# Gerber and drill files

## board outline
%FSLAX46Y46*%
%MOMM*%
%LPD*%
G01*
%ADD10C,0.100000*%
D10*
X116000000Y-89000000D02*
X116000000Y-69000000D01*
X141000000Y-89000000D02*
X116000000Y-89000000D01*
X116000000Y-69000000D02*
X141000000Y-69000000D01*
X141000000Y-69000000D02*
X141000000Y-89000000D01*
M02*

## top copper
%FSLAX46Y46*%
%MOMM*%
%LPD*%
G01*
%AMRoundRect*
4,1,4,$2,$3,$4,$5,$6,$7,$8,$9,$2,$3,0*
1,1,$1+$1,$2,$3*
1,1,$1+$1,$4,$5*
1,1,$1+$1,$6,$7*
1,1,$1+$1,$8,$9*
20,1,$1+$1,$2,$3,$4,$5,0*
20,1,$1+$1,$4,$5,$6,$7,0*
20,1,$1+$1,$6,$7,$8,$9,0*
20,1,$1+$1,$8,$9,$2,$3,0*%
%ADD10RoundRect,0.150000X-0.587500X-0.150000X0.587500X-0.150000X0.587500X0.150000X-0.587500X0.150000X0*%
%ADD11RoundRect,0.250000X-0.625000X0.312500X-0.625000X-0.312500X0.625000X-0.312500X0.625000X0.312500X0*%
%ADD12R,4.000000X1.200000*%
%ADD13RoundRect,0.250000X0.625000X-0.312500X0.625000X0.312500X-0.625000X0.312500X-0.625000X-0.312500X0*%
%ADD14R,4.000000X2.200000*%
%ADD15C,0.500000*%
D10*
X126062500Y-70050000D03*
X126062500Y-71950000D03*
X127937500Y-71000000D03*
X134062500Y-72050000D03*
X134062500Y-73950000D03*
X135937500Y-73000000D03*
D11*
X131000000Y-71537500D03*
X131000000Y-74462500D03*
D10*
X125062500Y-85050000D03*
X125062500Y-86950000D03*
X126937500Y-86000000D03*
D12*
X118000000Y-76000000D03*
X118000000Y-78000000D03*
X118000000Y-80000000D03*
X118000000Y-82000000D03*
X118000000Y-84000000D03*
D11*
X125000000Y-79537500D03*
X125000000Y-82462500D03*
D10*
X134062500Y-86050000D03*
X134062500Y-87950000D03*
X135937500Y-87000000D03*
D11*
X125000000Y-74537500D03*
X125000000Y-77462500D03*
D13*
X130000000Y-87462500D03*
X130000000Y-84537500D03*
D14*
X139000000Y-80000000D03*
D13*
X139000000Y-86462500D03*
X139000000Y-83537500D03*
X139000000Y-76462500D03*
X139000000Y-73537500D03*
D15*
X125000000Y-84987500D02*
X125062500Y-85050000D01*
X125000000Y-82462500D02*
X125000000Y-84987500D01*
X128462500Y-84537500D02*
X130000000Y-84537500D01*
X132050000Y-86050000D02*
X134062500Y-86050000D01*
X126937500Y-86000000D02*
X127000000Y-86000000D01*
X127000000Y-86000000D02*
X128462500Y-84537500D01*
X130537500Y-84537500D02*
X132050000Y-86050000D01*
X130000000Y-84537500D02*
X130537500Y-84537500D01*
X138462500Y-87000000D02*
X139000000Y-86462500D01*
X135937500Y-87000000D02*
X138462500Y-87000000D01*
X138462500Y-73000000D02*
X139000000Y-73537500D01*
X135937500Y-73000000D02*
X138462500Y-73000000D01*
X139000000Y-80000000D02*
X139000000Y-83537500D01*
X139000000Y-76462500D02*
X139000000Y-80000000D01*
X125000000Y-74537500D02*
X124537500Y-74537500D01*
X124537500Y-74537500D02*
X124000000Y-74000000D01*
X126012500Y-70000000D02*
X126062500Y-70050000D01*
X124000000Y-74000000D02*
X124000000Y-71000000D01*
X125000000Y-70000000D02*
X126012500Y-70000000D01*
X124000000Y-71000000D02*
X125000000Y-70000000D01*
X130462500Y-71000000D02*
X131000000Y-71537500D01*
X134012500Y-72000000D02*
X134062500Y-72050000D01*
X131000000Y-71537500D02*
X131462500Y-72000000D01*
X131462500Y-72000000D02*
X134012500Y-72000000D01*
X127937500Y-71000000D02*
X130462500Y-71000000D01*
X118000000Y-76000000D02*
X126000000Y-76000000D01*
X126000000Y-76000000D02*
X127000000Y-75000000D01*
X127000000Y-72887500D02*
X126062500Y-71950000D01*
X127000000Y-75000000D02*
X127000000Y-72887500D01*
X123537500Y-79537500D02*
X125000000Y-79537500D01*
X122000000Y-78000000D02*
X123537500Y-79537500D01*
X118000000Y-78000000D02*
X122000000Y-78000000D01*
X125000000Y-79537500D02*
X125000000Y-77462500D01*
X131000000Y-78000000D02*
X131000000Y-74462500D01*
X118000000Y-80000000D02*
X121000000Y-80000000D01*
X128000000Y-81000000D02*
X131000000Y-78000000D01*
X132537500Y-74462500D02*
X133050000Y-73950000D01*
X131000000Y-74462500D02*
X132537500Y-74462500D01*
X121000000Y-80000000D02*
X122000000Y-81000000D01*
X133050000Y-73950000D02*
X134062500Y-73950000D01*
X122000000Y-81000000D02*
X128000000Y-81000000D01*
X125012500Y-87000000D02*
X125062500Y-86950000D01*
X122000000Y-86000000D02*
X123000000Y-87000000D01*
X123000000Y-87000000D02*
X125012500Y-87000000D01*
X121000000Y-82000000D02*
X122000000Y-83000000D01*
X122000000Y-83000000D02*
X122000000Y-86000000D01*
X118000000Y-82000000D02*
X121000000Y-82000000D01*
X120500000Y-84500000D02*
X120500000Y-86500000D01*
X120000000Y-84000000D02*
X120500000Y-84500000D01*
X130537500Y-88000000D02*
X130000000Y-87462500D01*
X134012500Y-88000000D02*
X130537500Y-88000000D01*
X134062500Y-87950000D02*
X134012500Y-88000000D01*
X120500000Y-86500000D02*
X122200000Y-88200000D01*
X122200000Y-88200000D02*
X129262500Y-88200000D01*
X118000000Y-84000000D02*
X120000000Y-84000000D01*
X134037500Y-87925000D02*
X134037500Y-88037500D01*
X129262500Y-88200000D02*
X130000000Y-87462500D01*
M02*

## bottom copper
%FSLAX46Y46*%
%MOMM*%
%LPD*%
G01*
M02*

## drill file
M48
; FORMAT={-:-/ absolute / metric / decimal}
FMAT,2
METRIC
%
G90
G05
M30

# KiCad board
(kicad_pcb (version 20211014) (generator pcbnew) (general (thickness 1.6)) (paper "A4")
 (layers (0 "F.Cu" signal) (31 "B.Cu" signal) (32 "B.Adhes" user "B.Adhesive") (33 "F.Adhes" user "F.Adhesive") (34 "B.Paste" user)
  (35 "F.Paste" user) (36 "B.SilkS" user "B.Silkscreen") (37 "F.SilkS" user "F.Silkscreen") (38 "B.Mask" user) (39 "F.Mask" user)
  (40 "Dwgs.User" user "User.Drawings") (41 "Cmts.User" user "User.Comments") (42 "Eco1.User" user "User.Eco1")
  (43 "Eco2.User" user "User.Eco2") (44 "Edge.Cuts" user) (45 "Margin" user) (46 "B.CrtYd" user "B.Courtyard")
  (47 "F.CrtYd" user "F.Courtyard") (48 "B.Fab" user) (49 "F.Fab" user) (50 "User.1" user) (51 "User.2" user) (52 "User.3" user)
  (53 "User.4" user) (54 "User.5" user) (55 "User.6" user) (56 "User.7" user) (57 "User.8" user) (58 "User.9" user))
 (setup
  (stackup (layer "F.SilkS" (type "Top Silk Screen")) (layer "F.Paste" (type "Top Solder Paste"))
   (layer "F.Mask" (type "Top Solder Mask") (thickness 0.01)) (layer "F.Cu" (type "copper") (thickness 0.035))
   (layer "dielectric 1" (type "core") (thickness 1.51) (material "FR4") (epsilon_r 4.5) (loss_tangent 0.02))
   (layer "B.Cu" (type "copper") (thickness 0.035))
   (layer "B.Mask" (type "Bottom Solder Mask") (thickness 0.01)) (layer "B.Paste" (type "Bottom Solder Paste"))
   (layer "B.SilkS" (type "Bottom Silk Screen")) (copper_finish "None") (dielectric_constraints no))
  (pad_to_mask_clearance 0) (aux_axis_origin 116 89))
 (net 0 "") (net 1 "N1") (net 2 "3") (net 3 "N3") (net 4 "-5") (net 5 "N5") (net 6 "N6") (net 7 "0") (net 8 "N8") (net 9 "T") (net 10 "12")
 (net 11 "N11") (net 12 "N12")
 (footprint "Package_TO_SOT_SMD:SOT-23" (layer "F.Cu") (at 127 71)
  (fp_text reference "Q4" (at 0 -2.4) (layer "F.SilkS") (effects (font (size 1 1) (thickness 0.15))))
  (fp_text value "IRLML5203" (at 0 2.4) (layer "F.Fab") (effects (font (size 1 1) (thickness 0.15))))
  (pad "1" smd roundrect (at -0.9375 -0.95) (size 1.475 0.6) (layers "F.Cu" "F.Paste" "F.Mask") (roundrect_rratio 0.25) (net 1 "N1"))
  (pad "2" smd roundrect (at -0.9375 0.95) (size 1.475 0.6) (layers "F.Cu" "F.Paste" "F.Mask") (roundrect_rratio 0.25) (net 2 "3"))
  (pad "3" smd roundrect (at 0.9375 0) (size 1.475 0.6) (layers "F.Cu" "F.Paste" "F.Mask") (roundrect_rratio 0.25) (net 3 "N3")))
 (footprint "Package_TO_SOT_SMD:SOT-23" (layer "F.Cu") (at 135 73)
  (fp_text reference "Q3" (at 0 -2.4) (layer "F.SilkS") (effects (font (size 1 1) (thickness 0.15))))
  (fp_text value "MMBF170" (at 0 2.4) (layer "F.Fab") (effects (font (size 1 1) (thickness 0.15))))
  (pad "1" smd roundrect (at -0.9375 -0.95) (size 1.475 0.6) (layers "F.Cu" "F.Paste" "F.Mask") (roundrect_rratio 0.25) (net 3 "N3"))
  (pad "2" smd roundrect (at -0.9375 0.95) (size 1.475 0.6) (layers "F.Cu" "F.Paste" "F.Mask") (roundrect_rratio 0.25) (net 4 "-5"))
  (pad "3" smd roundrect (at 0.9375 0) (size 1.475 0.6) (layers "F.Cu" "F.Paste" "F.Mask") (roundrect_rratio 0.25) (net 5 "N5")))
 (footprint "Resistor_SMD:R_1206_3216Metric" (layer "F.Cu") (at 131 73 -90)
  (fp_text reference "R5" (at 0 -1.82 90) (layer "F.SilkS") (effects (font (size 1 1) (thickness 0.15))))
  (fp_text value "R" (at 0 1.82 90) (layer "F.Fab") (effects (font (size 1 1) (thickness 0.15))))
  (pad "1" smd roundrect (at -1.4625 0 270) (size 1.125 1.75) (layers "F.Cu" "F.Paste" "F.Mask") (roundrect_rratio 0.2222222222)
   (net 3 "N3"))
  (pad "2" smd roundrect (at 1.4625 0 270) (size 1.125 1.75) (layers "F.Cu" "F.Paste" "F.Mask") (roundrect_rratio 0.2222222222) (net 4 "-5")))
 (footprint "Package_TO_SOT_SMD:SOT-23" (layer "F.Cu") (at 126 86)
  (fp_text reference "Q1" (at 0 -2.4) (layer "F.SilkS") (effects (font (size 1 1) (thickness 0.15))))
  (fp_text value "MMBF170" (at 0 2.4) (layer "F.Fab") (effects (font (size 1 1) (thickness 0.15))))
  (pad "1" smd roundrect (at -0.9375 -0.95) (size 1.475 0.6) (layers "F.Cu" "F.Paste" "F.Mask") (roundrect_rratio 0.25) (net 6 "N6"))
  (pad "2" smd roundrect (at -0.9375 0.95) (size 1.475 0.6) (layers "F.Cu" "F.Paste" "F.Mask") (roundrect_rratio 0.25) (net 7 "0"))
  (pad "3" smd roundrect (at 0.9375 0) (size 1.475 0.6) (layers "F.Cu" "F.Paste" "F.Mask") (roundrect_rratio 0.25) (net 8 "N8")))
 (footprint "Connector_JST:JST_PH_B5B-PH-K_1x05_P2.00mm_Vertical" (layer "F.Cu") (at 118 76 -90)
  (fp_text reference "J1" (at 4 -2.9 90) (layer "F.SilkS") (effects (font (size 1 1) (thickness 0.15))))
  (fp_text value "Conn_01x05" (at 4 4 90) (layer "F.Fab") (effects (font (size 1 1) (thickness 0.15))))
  (pad "1" smd rect (at 0 0 270) (size 1.2 4) (layers "F.Cu" "F.Paste" "F.Mask") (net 2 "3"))
  (pad "2" smd rect (at 2 0 270) (size 1.2 4) (layers "F.Cu" "F.Paste" "F.Mask") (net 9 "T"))
  (pad "3" smd rect (at 4 0 270) (size 1.2 4) (layers "F.Cu" "F.Paste" "F.Mask") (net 4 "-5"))
  (pad "4" smd rect (at 6 0 270) (size 1.2 4) (layers "F.Cu" "F.Paste" "F.Mask") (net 7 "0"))
  (pad "5" smd rect (at 8 0 270) (size 1.2 4) (layers "F.Cu" "F.Paste" "F.Mask") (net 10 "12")))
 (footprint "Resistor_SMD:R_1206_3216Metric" (layer "F.Cu") (at 125 81 -90)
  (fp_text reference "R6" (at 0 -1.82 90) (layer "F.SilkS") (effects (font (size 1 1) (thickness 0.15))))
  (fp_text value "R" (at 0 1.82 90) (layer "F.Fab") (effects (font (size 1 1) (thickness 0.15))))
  (pad "1" smd roundrect (at -1.4625 0 270) (size 1.125 1.75) (layers "F.Cu" "F.Paste" "F.Mask") (roundrect_rratio 0.2222222222) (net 9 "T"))
  (pad "2" smd roundrect (at 1.4625 0 270) (size 1.125 1.75) (layers "F.Cu" "F.Paste" "F.Mask") (roundrect_rratio 0.2222222222) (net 6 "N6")))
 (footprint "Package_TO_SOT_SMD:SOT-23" (layer "F.Cu") (at 135 87)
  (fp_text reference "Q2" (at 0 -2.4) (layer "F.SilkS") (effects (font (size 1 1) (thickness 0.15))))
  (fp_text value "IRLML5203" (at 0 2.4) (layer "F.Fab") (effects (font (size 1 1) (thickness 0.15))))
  (pad "1" smd roundrect (at -0.9375 -0.95) (size 1.475 0.6) (layers "F.Cu" "F.Paste" "F.Mask") (roundrect_rratio 0.25) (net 8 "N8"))
  (pad "2" smd roundrect (at -0.9375 0.95) (size 1.475 0.6) (layers "F.Cu" "F.Paste" "F.Mask") (roundrect_rratio 0.25) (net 10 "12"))
  (pad "3" smd roundrect (at 0.9375 0) (size 1.475 0.6) (layers "F.Cu" "F.Paste" "F.Mask") (roundrect_rratio 0.25) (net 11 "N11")))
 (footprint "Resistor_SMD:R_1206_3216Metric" (layer "F.Cu") (at 125 76 -90)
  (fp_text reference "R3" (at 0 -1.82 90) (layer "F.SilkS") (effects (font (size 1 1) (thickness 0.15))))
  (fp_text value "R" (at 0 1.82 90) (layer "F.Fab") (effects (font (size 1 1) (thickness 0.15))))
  (pad "1" smd roundrect (at -1.4625 0 270) (size 1.125 1.75) (layers "F.Cu" "F.Paste" "F.Mask") (roundrect_rratio 0.2222222222)
   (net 1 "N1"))
  (pad "2" smd roundrect (at 1.4625 0 270) (size 1.125 1.75) (layers "F.Cu" "F.Paste" "F.Mask") (roundrect_rratio 0.2222222222) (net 9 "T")))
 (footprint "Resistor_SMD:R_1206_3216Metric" (layer "F.Cu") (at 130 86 90)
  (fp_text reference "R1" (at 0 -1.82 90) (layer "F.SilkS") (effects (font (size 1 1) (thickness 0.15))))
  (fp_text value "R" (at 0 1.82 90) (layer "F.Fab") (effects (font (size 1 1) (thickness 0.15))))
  (pad "1" smd roundrect (at -1.4625 0 90) (size 1.125 1.75) (layers "F.Cu" "F.Paste" "F.Mask") (roundrect_rratio 0.2222222222)
   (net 10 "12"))
  (pad "2" smd roundrect (at 1.4625 0 90) (size 1.125 1.75) (layers "F.Cu" "F.Paste" "F.Mask") (roundrect_rratio 0.2222222222) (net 8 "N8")))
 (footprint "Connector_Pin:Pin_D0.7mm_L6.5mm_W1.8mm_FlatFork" (layer "F.Cu") (at 139 80)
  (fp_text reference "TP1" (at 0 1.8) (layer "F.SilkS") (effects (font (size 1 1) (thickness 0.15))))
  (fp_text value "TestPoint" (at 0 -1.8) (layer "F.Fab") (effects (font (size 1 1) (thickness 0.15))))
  (pad "1" smd rect (at 0 0) (size 4 2.2) (layers "F.Cu" "F.Paste" "F.Mask") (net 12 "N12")))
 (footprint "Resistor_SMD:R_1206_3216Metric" (layer "F.Cu") (at 139 85 90)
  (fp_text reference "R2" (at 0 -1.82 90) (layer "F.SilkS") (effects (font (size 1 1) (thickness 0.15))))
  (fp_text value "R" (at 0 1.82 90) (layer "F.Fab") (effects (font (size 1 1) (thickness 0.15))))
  (pad "1" smd roundrect (at -1.4625 0 90) (size 1.125 1.75) (layers "F.Cu" "F.Paste" "F.Mask") (roundrect_rratio 0.2222222222)
   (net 11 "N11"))
  (pad "2" smd roundrect (at 1.4625 0 90) (size 1.125 1.75) (layers "F.Cu" "F.Paste" "F.Mask") (roundrect_rratio 0.2222222222)
   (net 12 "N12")))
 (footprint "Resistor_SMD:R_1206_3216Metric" (layer "F.Cu") (at 139 75 90)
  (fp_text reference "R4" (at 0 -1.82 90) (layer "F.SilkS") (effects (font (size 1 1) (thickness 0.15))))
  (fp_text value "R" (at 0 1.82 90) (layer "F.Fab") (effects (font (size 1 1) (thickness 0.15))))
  (pad "1" smd roundrect (at -1.4625 0 90) (size 1.125 1.75) (layers "F.Cu" "F.Paste" "F.Mask") (roundrect_rratio 0.2222222222)
   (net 12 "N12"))
  (pad "2" smd roundrect (at 1.4625 0 90) (size 1.125 1.75) (layers "F.Cu" "F.Paste" "F.Mask") (roundrect_rratio 0.2222222222) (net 5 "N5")))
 (gr_line (start 116 89) (end 116 69) (layer "Edge.Cuts") (width 0.1))
 (gr_line (start 141 89) (end 116 89) (layer "Edge.Cuts") (width 0.1))
 (gr_line (start 116 69) (end 141 69) (layer "Edge.Cuts") (width 0.1))
 (gr_line (start 141 69) (end 141 89) (layer "Edge.Cuts") (width 0.1))
 (segment (start 125 84.9875) (end 125.0625 85.05) (width 0.5) (layer "F.Cu") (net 6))
 (segment (start 125 82.4625) (end 125 84.9875) (width 0.5) (layer "F.Cu") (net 6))
 (segment (start 128.4625 84.5375) (end 130 84.5375) (width 0.5) (layer "F.Cu") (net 8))
 (segment (start 132.05 86.05) (end 134.0625 86.05) (width 0.5) (layer "F.Cu") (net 8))
 (segment (start 126.9375 86) (end 127 86) (width 0.5) (layer "F.Cu") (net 8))
 (segment (start 127 86) (end 128.4625 84.5375) (width 0.5) (layer "F.Cu") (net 8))
 (segment (start 130.5375 84.5375) (end 132.05 86.05) (width 0.5) (layer "F.Cu") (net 8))
 (segment (start 130 84.5375) (end 130.5375 84.5375) (width 0.5) (layer "F.Cu") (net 8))
 (segment (start 138.4625 87) (end 139 86.4625) (width 0.5) (layer "F.Cu") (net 11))
 (segment (start 135.9375 87) (end 138.4625 87) (width 0.5) (layer "F.Cu") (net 11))
 (segment (start 138.4625 73) (end 139 73.5375) (width 0.5) (layer "F.Cu") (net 5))
 (segment (start 135.9375 73) (end 138.4625 73) (width 0.5) (layer "F.Cu") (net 5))
 (segment (start 139 80) (end 139 83.5375) (width 0.5) (layer "F.Cu") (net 12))
 (segment (start 139 76.4625) (end 139 80) (width 0.5) (layer "F.Cu") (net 12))
 (segment (start 125 74.5375) (end 124.5375 74.5375) (width 0.5) (layer "F.Cu") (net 1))
 (segment (start 124.5375 74.5375) (end 124 74) (width 0.5) (layer "F.Cu") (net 1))
 (segment (start 126.0125 70) (end 126.0625 70.05) (width 0.5) (layer "F.Cu") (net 1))
 (segment (start 124 74) (end 124 71) (width 0.5) (layer "F.Cu") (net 1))
 (segment (start 125 70) (end 126.0125 70) (width 0.5) (layer "F.Cu") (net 1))
 (segment (start 124 71) (end 125 70) (width 0.5) (layer "F.Cu") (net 1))
 (segment (start 130.4625 71) (end 131 71.5375) (width 0.5) (layer "F.Cu") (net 3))
 (segment (start 134.0125 72) (end 134.0625 72.05) (width 0.5) (layer "F.Cu") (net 3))
 (segment (start 131 71.5375) (end 131.4625 72) (width 0.5) (layer "F.Cu") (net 3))
 (segment (start 131.4625 72) (end 134.0125 72) (width 0.5) (layer "F.Cu") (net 3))
 (segment (start 127.9375 71) (end 130.4625 71) (width 0.5) (layer "F.Cu") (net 3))
 (segment (start 118 76) (end 126 76) (width 0.5) (layer "F.Cu") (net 2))
 (segment (start 126 76) (end 127 75) (width 0.5) (layer "F.Cu") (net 2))
 (segment (start 127 72.8875) (end 126.0625 71.95) (width 0.5) (layer "F.Cu") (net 2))
 (segment (start 127 75) (end 127 72.8875) (width 0.5) (layer "F.Cu") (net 2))
 (segment (start 123.5375 79.5375) (end 125 79.5375) (width 0.5) (layer "F.Cu") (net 9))
 (segment (start 122 78) (end 123.5375 79.5375) (width 0.5) (layer "F.Cu") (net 9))
 (segment (start 118 78) (end 122 78) (width 0.5) (layer "F.Cu") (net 9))
 (segment (start 125 79.5375) (end 125 77.4625) (width 0.5) (layer "F.Cu") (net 9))
 (segment (start 131 78) (end 131 74.4625) (width 0.5) (layer "F.Cu") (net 4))
 (segment (start 118 80) (end 121 80) (width 0.5) (layer "F.Cu") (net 4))
 (segment (start 128 81) (end 131 78) (width 0.5) (layer "F.Cu") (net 4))
 (segment (start 132.5375 74.4625) (end 133.05 73.95) (width 0.5) (layer "F.Cu") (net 4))
 (segment (start 131 74.4625) (end 132.5375 74.4625) (width 0.5) (layer "F.Cu") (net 4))
 (segment (start 121 80) (end 122 81) (width 0.5) (layer "F.Cu") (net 4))
 (segment (start 133.05 73.95) (end 134.0625 73.95) (width 0.5) (layer "F.Cu") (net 4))
 (segment (start 122 81) (end 128 81) (width 0.5) (layer "F.Cu") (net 4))
 (segment (start 125.0125 87) (end 125.0625 86.95) (width 0.5) (layer "F.Cu") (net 7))
 (segment (start 122 86) (end 123 87) (width 0.5) (layer "F.Cu") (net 7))
 (segment (start 123 87) (end 125.0125 87) (width 0.5) (layer "F.Cu") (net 7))
 (segment (start 121 82) (end 122 83) (width 0.5) (layer "F.Cu") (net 7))
 (segment (start 122 83) (end 122 86) (width 0.5) (layer "F.Cu") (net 7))
 (segment (start 118 82) (end 121 82) (width 0.5) (layer "F.Cu") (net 7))
 (segment (start 120.5 84.5) (end 120.5 86.5) (width 0.5) (layer "F.Cu") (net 10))
 (segment (start 120 84) (end 120.5 84.5) (width 0.5) (layer "F.Cu") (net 10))
 (segment (start 130.5375 88) (end 130 87.4625) (width 0.5) (layer "F.Cu") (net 10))
 (segment (start 134.0125 88) (end 130.5375 88) (width 0.5) (layer "F.Cu") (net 10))
 (segment (start 134.0625 87.95) (end 134.0125 88) (width 0.5) (layer "F.Cu") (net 10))
 (segment (start 120.5 86.5) (end 122.2 88.2) (width 0.5) (layer "F.Cu") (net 10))
 (segment (start 122.2 88.2) (end 129.2625 88.2) (width 0.5) (layer "F.Cu") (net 10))
 (segment (start 118 84) (end 120 84) (width 0.5) (layer "F.Cu") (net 10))
 (segment (start 134.0375 87.925) (end 134.0375 88.0375) (width 0.5) (layer "F.Cu") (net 10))
 (segment (start 129.2625 88.2) (end 130 87.4625) (width 0.5) (layer "F.Cu") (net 10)))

